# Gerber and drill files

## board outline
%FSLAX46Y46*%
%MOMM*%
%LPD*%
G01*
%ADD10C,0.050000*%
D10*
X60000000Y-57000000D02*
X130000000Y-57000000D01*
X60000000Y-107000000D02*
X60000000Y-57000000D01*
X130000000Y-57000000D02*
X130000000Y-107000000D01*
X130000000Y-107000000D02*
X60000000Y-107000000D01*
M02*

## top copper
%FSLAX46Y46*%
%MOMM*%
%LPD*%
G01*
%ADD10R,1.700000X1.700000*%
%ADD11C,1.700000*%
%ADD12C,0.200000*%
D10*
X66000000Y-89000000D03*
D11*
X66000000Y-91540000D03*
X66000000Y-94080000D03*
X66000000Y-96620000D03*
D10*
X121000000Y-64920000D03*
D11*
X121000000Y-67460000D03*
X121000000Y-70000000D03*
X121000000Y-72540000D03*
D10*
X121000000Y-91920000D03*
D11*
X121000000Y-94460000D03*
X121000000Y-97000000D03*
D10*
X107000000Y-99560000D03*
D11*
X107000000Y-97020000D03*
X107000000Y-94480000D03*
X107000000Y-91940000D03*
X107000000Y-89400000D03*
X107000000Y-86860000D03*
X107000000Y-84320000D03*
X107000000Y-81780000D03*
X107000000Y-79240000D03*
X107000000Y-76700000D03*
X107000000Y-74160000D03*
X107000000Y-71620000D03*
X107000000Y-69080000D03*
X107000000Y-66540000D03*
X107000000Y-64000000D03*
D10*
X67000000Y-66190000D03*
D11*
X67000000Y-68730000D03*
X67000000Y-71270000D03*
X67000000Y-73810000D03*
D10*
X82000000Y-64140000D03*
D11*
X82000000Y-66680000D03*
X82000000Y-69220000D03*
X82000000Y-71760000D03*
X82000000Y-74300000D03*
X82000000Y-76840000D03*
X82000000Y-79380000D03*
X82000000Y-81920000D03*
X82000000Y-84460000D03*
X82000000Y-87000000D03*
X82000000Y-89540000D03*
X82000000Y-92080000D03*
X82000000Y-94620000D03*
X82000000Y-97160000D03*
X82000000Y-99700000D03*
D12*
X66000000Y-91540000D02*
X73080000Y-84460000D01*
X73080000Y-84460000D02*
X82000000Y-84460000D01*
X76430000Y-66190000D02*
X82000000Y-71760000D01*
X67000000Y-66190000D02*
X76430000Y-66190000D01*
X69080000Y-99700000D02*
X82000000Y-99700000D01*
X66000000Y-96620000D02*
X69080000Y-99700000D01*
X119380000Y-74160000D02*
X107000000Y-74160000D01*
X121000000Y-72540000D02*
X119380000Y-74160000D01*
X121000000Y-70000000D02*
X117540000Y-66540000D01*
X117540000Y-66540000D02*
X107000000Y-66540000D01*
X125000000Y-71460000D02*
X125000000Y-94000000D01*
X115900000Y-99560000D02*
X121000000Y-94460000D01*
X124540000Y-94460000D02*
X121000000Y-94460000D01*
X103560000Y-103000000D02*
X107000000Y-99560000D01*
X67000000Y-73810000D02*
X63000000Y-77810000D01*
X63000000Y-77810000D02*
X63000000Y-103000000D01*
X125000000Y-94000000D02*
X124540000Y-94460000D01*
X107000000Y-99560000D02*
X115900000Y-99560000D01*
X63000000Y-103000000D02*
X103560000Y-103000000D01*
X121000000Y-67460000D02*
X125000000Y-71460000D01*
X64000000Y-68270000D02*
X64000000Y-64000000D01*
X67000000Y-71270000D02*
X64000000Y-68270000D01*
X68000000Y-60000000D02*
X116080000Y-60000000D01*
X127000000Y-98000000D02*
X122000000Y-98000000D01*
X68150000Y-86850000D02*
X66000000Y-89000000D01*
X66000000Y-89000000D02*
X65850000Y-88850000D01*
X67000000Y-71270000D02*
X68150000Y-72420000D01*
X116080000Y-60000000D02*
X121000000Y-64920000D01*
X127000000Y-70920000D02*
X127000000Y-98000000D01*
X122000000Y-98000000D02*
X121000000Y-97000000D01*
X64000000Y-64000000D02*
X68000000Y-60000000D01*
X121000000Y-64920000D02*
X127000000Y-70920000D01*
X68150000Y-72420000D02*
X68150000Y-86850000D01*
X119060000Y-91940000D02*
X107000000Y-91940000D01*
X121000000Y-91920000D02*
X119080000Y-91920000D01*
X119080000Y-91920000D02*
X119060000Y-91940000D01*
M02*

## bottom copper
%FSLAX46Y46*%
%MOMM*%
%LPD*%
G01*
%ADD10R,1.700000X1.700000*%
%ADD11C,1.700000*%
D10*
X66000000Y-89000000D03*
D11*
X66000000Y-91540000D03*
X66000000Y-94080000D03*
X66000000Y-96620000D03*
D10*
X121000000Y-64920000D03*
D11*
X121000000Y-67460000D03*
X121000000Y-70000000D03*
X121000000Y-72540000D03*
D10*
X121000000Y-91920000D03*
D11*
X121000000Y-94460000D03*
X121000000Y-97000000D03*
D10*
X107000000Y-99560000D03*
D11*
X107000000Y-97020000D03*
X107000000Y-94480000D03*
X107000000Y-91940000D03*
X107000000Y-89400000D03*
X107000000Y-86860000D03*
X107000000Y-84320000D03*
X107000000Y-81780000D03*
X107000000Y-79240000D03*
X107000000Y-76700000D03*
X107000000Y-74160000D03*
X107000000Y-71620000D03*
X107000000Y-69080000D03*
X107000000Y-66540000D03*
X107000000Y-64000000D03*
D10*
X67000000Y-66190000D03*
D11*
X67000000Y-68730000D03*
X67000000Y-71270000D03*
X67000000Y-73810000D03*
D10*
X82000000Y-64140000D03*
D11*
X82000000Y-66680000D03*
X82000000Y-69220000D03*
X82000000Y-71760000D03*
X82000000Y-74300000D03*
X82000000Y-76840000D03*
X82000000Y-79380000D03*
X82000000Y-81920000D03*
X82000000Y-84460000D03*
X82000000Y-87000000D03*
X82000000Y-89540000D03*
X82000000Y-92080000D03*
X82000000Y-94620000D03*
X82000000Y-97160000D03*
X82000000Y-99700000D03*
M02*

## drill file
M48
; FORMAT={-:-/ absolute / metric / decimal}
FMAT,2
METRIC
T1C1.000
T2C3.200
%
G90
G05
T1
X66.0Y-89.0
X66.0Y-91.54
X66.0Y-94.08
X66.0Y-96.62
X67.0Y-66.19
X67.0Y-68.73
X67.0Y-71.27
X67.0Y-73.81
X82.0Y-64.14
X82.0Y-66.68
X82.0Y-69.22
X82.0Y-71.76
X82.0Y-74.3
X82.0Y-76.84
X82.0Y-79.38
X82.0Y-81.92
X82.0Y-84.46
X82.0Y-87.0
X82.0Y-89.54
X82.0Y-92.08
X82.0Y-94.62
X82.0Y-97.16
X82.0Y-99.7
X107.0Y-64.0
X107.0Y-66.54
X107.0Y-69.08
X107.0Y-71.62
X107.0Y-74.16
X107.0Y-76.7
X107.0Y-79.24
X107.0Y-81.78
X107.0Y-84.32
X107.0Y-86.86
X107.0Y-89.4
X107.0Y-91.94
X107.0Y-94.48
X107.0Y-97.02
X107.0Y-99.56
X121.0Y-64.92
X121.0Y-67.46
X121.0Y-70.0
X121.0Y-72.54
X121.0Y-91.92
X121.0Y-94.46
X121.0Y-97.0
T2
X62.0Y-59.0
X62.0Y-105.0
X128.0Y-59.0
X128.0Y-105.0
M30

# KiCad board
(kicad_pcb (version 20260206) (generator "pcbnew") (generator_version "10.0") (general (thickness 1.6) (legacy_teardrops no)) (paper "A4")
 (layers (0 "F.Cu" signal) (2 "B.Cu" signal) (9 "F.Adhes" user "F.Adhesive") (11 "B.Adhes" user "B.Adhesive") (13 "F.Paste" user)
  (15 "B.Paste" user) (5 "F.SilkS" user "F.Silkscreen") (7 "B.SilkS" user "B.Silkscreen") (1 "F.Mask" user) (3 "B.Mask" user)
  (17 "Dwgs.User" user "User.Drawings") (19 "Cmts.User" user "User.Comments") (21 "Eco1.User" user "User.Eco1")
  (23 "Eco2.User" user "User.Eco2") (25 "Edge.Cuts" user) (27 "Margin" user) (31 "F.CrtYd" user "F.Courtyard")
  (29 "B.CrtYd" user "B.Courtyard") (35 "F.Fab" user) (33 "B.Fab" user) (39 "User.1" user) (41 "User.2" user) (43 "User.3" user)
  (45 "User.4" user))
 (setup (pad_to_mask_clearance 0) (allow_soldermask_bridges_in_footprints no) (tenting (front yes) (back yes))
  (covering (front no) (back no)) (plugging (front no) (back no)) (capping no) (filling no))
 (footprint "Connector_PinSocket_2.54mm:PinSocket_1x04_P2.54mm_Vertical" (layer "F.Cu") (at 66 89)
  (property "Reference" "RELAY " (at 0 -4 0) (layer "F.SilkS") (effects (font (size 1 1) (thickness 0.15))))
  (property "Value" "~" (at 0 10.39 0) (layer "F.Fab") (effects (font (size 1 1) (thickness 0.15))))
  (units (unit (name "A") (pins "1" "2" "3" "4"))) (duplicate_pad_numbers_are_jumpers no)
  (pad "1" thru_hole rect (at 0 0) (size 1.7 1.7) (drill 1) (layers "*.Cu" "*.Mask") (remove_unused_layers no) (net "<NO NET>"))
  (pad "2" thru_hole circle (at 0 2.54) (size 1.7 1.7) (drill 1) (layers "*.Cu" "*.Mask") (remove_unused_layers no) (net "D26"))
  (pad "3" thru_hole circle (at 0 5.08) (size 1.7 1.7) (drill 1) (layers "*.Cu" "*.Mask") (remove_unused_layers no)
   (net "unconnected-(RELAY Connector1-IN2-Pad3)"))
  (pad "4" thru_hole circle (at 0 7.62) (size 1.7 1.7) (drill 1) (layers "*.Cu" "*.Mask") (remove_unused_layers no) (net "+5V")))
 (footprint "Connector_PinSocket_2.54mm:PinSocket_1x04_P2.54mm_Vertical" (layer "F.Cu") (at 121 64.92)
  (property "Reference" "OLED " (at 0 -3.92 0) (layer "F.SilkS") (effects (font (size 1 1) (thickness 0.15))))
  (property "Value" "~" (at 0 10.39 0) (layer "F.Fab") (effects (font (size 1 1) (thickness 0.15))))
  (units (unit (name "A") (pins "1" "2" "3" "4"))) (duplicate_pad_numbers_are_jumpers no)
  (pad "1" thru_hole rect (at 0 0) (size 1.7 1.7) (drill 1) (layers "*.Cu" "*.Mask") (remove_unused_layers no) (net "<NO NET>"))
  (pad "2" thru_hole circle (at 0 2.54) (size 1.7 1.7) (drill 1) (layers "*.Cu" "*.Mask") (remove_unused_layers no) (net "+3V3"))
  (pad "3" thru_hole circle (at 0 5.08) (size 1.7 1.7) (drill 1) (layers "*.Cu" "*.Mask") (remove_unused_layers no) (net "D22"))
  (pad "4" thru_hole circle (at 0 7.62) (size 1.7 1.7) (drill 1) (layers "*.Cu" "*.Mask") (remove_unused_layers no) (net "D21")))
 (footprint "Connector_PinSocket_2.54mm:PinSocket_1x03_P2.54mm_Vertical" (layer "F.Cu") (at 121 91.92)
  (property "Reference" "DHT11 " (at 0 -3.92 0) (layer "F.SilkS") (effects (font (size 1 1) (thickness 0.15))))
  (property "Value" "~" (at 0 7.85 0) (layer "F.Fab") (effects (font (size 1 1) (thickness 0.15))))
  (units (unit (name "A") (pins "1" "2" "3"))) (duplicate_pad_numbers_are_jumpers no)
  (pad "1" thru_hole rect (at 0 0) (size 1.7 1.7) (drill 1) (layers "*.Cu" "*.Mask") (remove_unused_layers no) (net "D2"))
  (pad "2" thru_hole circle (at 0 2.54) (size 1.7 1.7) (drill 1) (layers "*.Cu" "*.Mask") (remove_unused_layers no) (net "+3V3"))
  (pad "3" thru_hole circle (at 0 5.08) (size 1.7 1.7) (drill 1) (layers "*.Cu" "*.Mask") (remove_unused_layers no) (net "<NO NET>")))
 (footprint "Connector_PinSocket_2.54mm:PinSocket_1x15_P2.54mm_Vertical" (layer "F.Cu") (at 107 99.56 180)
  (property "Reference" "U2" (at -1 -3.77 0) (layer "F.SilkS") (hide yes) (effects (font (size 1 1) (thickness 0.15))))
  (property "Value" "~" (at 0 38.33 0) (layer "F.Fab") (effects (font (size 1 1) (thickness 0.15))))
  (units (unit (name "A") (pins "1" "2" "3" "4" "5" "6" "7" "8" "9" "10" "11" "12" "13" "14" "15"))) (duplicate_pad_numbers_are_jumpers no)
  (pad "1" thru_hole rect (at 0 0 180) (size 1.7 1.7) (drill 1) (layers "*.Cu" "*.Mask") (remove_unused_layers no) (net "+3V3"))
  (pad "2" thru_hole circle (at 0 2.54 180) (size 1.7 1.7) (drill 1) (layers "*.Cu" "*.Mask") (remove_unused_layers no) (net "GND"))
  (pad "3" thru_hole circle (at 0 5.08 180) (size 1.7 1.7) (drill 1) (layers "*.Cu" "*.Mask") (remove_unused_layers no)
   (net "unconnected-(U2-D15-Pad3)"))
  (pad "4" thru_hole circle (at 0 7.62 180) (size 1.7 1.7) (drill 1) (layers "*.Cu" "*.Mask") (remove_unused_layers no) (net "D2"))
  (pad "5" thru_hole circle (at 0 10.16 180) (size 1.7 1.7) (drill 1) (layers "*.Cu" "*.Mask") (remove_unused_layers no)
   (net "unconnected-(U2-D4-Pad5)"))
  (pad "6" thru_hole circle (at 0 12.7 180) (size 1.7 1.7) (drill 1) (layers "*.Cu" "*.Mask") (remove_unused_layers no)
   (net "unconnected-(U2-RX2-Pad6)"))
  (pad "7" thru_hole circle (at 0 15.24 180) (size 1.7 1.7) (drill 1) (layers "*.Cu" "*.Mask") (remove_unused_layers no)
   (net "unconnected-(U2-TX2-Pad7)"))
  (pad "8" thru_hole circle (at 0 17.78 180) (size 1.7 1.7) (drill 1) (layers "*.Cu" "*.Mask") (remove_unused_layers no)
   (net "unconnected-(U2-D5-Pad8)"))
  (pad "9" thru_hole circle (at 0 20.32 180) (size 1.7 1.7) (drill 1) (layers "*.Cu" "*.Mask") (remove_unused_layers no)
   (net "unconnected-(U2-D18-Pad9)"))
  (pad "10" thru_hole circle (at 0 22.86 180) (size 1.7 1.7) (drill 1) (layers "*.Cu" "*.Mask") (remove_unused_layers no)
   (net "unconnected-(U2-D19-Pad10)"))
  (pad "11" thru_hole circle (at 0 25.4 180) (size 1.7 1.7) (drill 1) (layers "*.Cu" "*.Mask") (remove_unused_layers no) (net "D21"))
  (pad "12" thru_hole circle (at 0 27.94 180) (size 1.7 1.7) (drill 1) (layers "*.Cu" "*.Mask") (remove_unused_layers no)
   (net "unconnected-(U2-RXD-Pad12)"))
  (pad "13" thru_hole circle (at 0 30.48 180) (size 1.7 1.7) (drill 1) (layers "*.Cu" "*.Mask") (remove_unused_layers no)
   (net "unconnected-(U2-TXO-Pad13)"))
  (pad "14" thru_hole circle (at 0 33.02 180) (size 1.7 1.7) (drill 1) (layers "*.Cu" "*.Mask") (remove_unused_layers no) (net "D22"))
  (pad "15" thru_hole circle (at 0 35.56 180) (size 1.7 1.7) (drill 1) (layers "*.Cu" "*.Mask") (remove_unused_layers no)
   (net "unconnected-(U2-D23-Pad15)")))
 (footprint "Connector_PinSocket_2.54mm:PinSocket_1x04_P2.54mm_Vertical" (layer "F.Cu") (at 67 66.19)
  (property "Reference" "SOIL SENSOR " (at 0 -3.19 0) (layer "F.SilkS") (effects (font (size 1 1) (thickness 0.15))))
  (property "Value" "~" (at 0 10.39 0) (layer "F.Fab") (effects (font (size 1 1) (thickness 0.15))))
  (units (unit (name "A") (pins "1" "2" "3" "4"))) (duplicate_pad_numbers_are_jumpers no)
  (pad "1" thru_hole rect (at 0 0) (size 1.7 1.7) (drill 1) (layers "*.Cu" "*.Mask") (remove_unused_layers no) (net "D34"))
  (pad "2" thru_hole circle (at 0 2.54) (size 1.7 1.7) (drill 1) (layers "*.Cu" "*.Mask") (remove_unused_layers no)
   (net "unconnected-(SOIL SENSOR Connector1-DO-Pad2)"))
  (pad "3" thru_hole circle (at 0 5.08) (size 1.7 1.7) (drill 1) (layers "*.Cu" "*.Mask") (remove_unused_layers no) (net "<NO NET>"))
  (pad "4" thru_hole circle (at 0 7.62) (size 1.7 1.7) (drill 1) (layers "*.Cu" "*.Mask") (remove_unused_layers no) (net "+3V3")))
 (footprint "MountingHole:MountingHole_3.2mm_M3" (layer "F.Cu") (at 128 59)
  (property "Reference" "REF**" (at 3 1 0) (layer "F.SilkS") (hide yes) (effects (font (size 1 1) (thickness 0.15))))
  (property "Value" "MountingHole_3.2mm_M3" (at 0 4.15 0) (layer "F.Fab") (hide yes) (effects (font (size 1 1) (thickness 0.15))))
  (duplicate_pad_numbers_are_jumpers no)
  (pad "" np_thru_hole circle (at 0 0) (size 3.2 3.2) (drill 3.2) (layers "*.Cu" "*.Mask")))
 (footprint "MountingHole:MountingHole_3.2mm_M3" (layer "F.Cu") (at 128 105)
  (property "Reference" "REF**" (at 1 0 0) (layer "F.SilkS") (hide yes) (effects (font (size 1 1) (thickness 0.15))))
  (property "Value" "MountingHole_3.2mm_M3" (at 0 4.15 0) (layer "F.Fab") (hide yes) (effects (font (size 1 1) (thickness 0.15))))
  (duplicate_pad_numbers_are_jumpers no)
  (pad "" np_thru_hole circle (at 0 0) (size 3.2 3.2) (drill 3.2) (layers "*.Cu" "*.Mask")))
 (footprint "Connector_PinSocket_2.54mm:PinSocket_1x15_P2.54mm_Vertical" (layer "F.Cu") (at 82 64.14)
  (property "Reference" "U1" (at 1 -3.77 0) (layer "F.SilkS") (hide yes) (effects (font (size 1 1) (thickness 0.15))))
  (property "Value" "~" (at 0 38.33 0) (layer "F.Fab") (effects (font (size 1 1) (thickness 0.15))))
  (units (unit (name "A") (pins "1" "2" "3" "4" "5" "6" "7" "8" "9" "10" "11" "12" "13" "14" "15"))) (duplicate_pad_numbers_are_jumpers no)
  (pad "1" thru_hole rect (at 0 0) (size 1.7 1.7) (drill 1) (layers "*.Cu" "*.Mask") (remove_unused_layers no)
   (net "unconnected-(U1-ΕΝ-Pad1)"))
  (pad "2" thru_hole circle (at 0 2.54) (size 1.7 1.7) (drill 1) (layers "*.Cu" "*.Mask") (remove_unused_layers no)
   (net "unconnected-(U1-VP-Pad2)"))
  (pad "3" thru_hole circle (at 0 5.08) (size 1.7 1.7) (drill 1) (layers "*.Cu" "*.Mask") (remove_unused_layers no)
   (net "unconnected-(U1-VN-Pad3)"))
  (pad "4" thru_hole circle (at 0 7.62) (size 1.7 1.7) (drill 1) (layers "*.Cu" "*.Mask") (remove_unused_layers no) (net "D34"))
  (pad "5" thru_hole circle (at 0 10.16) (size 1.7 1.7) (drill 1) (layers "*.Cu" "*.Mask") (remove_unused_layers no)
   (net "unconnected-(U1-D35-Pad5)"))
  (pad "6" thru_hole circle (at 0 12.7) (size 1.7 1.7) (drill 1) (layers "*.Cu" "*.Mask") (remove_unused_layers no)
   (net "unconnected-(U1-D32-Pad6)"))
  (pad "7" thru_hole circle (at 0 15.24) (size 1.7 1.7) (drill 1) (layers "*.Cu" "*.Mask") (remove_unused_layers no)
   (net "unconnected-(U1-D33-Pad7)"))
  (pad "8" thru_hole circle (at 0 17.78) (size 1.7 1.7) (drill 1) (layers "*.Cu" "*.Mask") (remove_unused_layers no)
   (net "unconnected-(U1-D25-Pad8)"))
  (pad "9" thru_hole circle (at 0 20.32) (size 1.7 1.7) (drill 1) (layers "*.Cu" "*.Mask") (remove_unused_layers no) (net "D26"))
  (pad "10" thru_hole circle (at 0 22.86) (size 1.7 1.7) (drill 1) (layers "*.Cu" "*.Mask") (remove_unused_layers no)
   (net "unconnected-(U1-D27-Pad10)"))
  (pad "11" thru_hole circle (at 0 25.4) (size 1.7 1.7) (drill 1) (layers "*.Cu" "*.Mask") (remove_unused_layers no)
   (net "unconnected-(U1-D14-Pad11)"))
  (pad "12" thru_hole circle (at 0 27.94) (size 1.7 1.7) (drill 1) (layers "*.Cu" "*.Mask") (remove_unused_layers no)
   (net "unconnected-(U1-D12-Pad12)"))
  (pad "13" thru_hole circle (at 0 30.48) (size 1.7 1.7) (drill 1) (layers "*.Cu" "*.Mask") (remove_unused_layers no)
   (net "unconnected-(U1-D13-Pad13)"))
  (pad "14" thru_hole circle (at 0 33.02) (size 1.7 1.7) (drill 1) (layers "*.Cu" "*.Mask") (remove_unused_layers no)
   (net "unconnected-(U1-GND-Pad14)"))
  (pad "15" thru_hole circle (at 0 35.56) (size 1.7 1.7) (drill 1) (layers "*.Cu" "*.Mask") (remove_unused_layers no) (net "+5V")))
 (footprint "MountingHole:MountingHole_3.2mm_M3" (layer "F.Cu") (at 62 105)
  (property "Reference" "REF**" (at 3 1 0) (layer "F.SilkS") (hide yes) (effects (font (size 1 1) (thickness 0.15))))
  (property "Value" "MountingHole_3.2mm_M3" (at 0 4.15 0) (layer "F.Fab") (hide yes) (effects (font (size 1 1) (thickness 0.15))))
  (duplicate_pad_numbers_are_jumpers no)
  (pad "" np_thru_hole circle (at 0 0) (size 3.2 3.2) (drill 3.2) (layers "*.Cu" "*.Mask")))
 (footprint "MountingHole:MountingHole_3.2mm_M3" (layer "F.Cu") (at 62 59)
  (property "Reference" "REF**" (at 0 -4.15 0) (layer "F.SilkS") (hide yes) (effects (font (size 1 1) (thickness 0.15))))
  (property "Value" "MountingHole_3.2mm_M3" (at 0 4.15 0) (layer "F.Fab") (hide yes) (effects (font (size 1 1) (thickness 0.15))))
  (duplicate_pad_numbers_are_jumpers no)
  (pad "" np_thru_hole circle (at 0 0) (size 3.2 3.2) (drill 3.2) (layers "*.Cu" "*.Mask")))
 (gr_line (start 60 57) (end 130 57) (stroke (width 0.05) (type default)) (layer "Edge.Cuts"))
 (gr_line (start 60 107) (end 60 57) (stroke (width 0.05) (type default)) (layer "Edge.Cuts"))
 (gr_line (start 130 57) (end 130 107) (stroke (width 0.05) (type default)) (layer "Edge.Cuts"))
 (gr_line (start 130 107) (end 60 107) (stroke (width 0.05) (type default)) (layer "Edge.Cuts"))
 (segment (start 66 91.54) (end 73.08 84.46) (width 0.2) (layer "F.Cu") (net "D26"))
 (segment (start 73.08 84.46) (end 82 84.46) (width 0.2) (layer "F.Cu") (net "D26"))
 (segment (start 76.43 66.19) (end 82 71.76) (width 0.2) (layer "F.Cu") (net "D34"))
 (segment (start 67 66.19) (end 76.43 66.19) (width 0.2) (layer "F.Cu") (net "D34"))
 (segment (start 69.08 99.7) (end 82 99.7) (width 0.2) (layer "F.Cu") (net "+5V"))
 (segment (start 66 96.62) (end 69.08 99.7) (width 0.2) (layer "F.Cu") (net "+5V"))
 (segment (start 119.38 74.16) (end 107 74.16) (width 0.2) (layer "F.Cu") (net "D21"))
 (segment (start 121 72.54) (end 119.38 74.16) (width 0.2) (layer "F.Cu") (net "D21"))
 (segment (start 121 70) (end 117.54 66.54) (width 0.2) (layer "F.Cu") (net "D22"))
 (segment (start 117.54 66.54) (end 107 66.54) (width 0.2) (layer "F.Cu") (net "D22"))
 (segment (start 125 71.46) (end 125 94) (width 0.2) (layer "F.Cu") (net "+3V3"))
 (segment (start 115.9 99.56) (end 121 94.46) (width 0.2) (layer "F.Cu") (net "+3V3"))
 (segment (start 124.54 94.46) (end 121 94.46) (width 0.2) (layer "F.Cu") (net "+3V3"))
 (segment (start 103.56 103) (end 107 99.56) (width 0.2) (layer "F.Cu") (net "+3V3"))
 (segment (start 67 73.81) (end 63 77.81) (width 0.2) (layer "F.Cu") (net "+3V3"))
 (segment (start 63 77.81) (end 63 103) (width 0.2) (layer "F.Cu") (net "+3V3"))
 (segment (start 125 94) (end 124.54 94.46) (width 0.2) (layer "F.Cu") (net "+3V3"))
 (segment (start 107 99.56) (end 115.9 99.56) (width 0.2) (layer "F.Cu") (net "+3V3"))
 (segment (start 63 103) (end 103.56 103) (width 0.2) (layer "F.Cu") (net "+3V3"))
 (segment (start 121 67.46) (end 125 71.46) (width 0.2) (layer "F.Cu") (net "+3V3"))
 (segment (start 64 68.27) (end 64 64) (width 0.2) (layer "F.Cu") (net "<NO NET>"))
 (segment (start 67 71.27) (end 64 68.27) (width 0.2) (layer "F.Cu") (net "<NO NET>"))
 (segment (start 68 60) (end 116.08 60) (width 0.2) (layer "F.Cu") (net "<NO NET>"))
 (segment (start 127 98) (end 122 98) (width 0.2) (layer "F.Cu") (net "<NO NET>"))
 (segment (start 68.15 86.85) (end 66 89) (width 0.2) (layer "F.Cu") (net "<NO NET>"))
 (segment (start 66 89) (end 65.85 88.85) (width 0.2) (layer "F.Cu") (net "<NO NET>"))
 (segment (start 67 71.27) (end 68.15 72.42) (width 0.2) (layer "F.Cu") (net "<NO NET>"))
 (segment (start 116.08 60) (end 121 64.92) (width 0.2) (layer "F.Cu") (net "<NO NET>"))
 (segment (start 127 70.92) (end 127 98) (width 0.2) (layer "F.Cu") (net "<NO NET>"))
 (segment (start 122 98) (end 121 97) (width 0.2) (layer "F.Cu") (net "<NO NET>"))
 (segment (start 64 64) (end 68 60) (width 0.2) (layer "F.Cu") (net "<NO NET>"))
 (segment (start 121 64.92) (end 127 70.92) (width 0.2) (layer "F.Cu") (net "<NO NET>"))
 (segment (start 68.15 72.42) (end 68.15 86.85) (width 0.2) (layer "F.Cu") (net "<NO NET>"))
 (segment (start 119.06 91.94) (end 107 91.94) (width 0.2) (layer "F.Cu") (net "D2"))
 (segment (start 121 91.92) (end 119.08 91.92) (width 0.2) (layer "F.Cu") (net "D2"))
 (segment (start 119.08 91.92) (end 119.06 91.94) (width 0.2) (layer "F.Cu") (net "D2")))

